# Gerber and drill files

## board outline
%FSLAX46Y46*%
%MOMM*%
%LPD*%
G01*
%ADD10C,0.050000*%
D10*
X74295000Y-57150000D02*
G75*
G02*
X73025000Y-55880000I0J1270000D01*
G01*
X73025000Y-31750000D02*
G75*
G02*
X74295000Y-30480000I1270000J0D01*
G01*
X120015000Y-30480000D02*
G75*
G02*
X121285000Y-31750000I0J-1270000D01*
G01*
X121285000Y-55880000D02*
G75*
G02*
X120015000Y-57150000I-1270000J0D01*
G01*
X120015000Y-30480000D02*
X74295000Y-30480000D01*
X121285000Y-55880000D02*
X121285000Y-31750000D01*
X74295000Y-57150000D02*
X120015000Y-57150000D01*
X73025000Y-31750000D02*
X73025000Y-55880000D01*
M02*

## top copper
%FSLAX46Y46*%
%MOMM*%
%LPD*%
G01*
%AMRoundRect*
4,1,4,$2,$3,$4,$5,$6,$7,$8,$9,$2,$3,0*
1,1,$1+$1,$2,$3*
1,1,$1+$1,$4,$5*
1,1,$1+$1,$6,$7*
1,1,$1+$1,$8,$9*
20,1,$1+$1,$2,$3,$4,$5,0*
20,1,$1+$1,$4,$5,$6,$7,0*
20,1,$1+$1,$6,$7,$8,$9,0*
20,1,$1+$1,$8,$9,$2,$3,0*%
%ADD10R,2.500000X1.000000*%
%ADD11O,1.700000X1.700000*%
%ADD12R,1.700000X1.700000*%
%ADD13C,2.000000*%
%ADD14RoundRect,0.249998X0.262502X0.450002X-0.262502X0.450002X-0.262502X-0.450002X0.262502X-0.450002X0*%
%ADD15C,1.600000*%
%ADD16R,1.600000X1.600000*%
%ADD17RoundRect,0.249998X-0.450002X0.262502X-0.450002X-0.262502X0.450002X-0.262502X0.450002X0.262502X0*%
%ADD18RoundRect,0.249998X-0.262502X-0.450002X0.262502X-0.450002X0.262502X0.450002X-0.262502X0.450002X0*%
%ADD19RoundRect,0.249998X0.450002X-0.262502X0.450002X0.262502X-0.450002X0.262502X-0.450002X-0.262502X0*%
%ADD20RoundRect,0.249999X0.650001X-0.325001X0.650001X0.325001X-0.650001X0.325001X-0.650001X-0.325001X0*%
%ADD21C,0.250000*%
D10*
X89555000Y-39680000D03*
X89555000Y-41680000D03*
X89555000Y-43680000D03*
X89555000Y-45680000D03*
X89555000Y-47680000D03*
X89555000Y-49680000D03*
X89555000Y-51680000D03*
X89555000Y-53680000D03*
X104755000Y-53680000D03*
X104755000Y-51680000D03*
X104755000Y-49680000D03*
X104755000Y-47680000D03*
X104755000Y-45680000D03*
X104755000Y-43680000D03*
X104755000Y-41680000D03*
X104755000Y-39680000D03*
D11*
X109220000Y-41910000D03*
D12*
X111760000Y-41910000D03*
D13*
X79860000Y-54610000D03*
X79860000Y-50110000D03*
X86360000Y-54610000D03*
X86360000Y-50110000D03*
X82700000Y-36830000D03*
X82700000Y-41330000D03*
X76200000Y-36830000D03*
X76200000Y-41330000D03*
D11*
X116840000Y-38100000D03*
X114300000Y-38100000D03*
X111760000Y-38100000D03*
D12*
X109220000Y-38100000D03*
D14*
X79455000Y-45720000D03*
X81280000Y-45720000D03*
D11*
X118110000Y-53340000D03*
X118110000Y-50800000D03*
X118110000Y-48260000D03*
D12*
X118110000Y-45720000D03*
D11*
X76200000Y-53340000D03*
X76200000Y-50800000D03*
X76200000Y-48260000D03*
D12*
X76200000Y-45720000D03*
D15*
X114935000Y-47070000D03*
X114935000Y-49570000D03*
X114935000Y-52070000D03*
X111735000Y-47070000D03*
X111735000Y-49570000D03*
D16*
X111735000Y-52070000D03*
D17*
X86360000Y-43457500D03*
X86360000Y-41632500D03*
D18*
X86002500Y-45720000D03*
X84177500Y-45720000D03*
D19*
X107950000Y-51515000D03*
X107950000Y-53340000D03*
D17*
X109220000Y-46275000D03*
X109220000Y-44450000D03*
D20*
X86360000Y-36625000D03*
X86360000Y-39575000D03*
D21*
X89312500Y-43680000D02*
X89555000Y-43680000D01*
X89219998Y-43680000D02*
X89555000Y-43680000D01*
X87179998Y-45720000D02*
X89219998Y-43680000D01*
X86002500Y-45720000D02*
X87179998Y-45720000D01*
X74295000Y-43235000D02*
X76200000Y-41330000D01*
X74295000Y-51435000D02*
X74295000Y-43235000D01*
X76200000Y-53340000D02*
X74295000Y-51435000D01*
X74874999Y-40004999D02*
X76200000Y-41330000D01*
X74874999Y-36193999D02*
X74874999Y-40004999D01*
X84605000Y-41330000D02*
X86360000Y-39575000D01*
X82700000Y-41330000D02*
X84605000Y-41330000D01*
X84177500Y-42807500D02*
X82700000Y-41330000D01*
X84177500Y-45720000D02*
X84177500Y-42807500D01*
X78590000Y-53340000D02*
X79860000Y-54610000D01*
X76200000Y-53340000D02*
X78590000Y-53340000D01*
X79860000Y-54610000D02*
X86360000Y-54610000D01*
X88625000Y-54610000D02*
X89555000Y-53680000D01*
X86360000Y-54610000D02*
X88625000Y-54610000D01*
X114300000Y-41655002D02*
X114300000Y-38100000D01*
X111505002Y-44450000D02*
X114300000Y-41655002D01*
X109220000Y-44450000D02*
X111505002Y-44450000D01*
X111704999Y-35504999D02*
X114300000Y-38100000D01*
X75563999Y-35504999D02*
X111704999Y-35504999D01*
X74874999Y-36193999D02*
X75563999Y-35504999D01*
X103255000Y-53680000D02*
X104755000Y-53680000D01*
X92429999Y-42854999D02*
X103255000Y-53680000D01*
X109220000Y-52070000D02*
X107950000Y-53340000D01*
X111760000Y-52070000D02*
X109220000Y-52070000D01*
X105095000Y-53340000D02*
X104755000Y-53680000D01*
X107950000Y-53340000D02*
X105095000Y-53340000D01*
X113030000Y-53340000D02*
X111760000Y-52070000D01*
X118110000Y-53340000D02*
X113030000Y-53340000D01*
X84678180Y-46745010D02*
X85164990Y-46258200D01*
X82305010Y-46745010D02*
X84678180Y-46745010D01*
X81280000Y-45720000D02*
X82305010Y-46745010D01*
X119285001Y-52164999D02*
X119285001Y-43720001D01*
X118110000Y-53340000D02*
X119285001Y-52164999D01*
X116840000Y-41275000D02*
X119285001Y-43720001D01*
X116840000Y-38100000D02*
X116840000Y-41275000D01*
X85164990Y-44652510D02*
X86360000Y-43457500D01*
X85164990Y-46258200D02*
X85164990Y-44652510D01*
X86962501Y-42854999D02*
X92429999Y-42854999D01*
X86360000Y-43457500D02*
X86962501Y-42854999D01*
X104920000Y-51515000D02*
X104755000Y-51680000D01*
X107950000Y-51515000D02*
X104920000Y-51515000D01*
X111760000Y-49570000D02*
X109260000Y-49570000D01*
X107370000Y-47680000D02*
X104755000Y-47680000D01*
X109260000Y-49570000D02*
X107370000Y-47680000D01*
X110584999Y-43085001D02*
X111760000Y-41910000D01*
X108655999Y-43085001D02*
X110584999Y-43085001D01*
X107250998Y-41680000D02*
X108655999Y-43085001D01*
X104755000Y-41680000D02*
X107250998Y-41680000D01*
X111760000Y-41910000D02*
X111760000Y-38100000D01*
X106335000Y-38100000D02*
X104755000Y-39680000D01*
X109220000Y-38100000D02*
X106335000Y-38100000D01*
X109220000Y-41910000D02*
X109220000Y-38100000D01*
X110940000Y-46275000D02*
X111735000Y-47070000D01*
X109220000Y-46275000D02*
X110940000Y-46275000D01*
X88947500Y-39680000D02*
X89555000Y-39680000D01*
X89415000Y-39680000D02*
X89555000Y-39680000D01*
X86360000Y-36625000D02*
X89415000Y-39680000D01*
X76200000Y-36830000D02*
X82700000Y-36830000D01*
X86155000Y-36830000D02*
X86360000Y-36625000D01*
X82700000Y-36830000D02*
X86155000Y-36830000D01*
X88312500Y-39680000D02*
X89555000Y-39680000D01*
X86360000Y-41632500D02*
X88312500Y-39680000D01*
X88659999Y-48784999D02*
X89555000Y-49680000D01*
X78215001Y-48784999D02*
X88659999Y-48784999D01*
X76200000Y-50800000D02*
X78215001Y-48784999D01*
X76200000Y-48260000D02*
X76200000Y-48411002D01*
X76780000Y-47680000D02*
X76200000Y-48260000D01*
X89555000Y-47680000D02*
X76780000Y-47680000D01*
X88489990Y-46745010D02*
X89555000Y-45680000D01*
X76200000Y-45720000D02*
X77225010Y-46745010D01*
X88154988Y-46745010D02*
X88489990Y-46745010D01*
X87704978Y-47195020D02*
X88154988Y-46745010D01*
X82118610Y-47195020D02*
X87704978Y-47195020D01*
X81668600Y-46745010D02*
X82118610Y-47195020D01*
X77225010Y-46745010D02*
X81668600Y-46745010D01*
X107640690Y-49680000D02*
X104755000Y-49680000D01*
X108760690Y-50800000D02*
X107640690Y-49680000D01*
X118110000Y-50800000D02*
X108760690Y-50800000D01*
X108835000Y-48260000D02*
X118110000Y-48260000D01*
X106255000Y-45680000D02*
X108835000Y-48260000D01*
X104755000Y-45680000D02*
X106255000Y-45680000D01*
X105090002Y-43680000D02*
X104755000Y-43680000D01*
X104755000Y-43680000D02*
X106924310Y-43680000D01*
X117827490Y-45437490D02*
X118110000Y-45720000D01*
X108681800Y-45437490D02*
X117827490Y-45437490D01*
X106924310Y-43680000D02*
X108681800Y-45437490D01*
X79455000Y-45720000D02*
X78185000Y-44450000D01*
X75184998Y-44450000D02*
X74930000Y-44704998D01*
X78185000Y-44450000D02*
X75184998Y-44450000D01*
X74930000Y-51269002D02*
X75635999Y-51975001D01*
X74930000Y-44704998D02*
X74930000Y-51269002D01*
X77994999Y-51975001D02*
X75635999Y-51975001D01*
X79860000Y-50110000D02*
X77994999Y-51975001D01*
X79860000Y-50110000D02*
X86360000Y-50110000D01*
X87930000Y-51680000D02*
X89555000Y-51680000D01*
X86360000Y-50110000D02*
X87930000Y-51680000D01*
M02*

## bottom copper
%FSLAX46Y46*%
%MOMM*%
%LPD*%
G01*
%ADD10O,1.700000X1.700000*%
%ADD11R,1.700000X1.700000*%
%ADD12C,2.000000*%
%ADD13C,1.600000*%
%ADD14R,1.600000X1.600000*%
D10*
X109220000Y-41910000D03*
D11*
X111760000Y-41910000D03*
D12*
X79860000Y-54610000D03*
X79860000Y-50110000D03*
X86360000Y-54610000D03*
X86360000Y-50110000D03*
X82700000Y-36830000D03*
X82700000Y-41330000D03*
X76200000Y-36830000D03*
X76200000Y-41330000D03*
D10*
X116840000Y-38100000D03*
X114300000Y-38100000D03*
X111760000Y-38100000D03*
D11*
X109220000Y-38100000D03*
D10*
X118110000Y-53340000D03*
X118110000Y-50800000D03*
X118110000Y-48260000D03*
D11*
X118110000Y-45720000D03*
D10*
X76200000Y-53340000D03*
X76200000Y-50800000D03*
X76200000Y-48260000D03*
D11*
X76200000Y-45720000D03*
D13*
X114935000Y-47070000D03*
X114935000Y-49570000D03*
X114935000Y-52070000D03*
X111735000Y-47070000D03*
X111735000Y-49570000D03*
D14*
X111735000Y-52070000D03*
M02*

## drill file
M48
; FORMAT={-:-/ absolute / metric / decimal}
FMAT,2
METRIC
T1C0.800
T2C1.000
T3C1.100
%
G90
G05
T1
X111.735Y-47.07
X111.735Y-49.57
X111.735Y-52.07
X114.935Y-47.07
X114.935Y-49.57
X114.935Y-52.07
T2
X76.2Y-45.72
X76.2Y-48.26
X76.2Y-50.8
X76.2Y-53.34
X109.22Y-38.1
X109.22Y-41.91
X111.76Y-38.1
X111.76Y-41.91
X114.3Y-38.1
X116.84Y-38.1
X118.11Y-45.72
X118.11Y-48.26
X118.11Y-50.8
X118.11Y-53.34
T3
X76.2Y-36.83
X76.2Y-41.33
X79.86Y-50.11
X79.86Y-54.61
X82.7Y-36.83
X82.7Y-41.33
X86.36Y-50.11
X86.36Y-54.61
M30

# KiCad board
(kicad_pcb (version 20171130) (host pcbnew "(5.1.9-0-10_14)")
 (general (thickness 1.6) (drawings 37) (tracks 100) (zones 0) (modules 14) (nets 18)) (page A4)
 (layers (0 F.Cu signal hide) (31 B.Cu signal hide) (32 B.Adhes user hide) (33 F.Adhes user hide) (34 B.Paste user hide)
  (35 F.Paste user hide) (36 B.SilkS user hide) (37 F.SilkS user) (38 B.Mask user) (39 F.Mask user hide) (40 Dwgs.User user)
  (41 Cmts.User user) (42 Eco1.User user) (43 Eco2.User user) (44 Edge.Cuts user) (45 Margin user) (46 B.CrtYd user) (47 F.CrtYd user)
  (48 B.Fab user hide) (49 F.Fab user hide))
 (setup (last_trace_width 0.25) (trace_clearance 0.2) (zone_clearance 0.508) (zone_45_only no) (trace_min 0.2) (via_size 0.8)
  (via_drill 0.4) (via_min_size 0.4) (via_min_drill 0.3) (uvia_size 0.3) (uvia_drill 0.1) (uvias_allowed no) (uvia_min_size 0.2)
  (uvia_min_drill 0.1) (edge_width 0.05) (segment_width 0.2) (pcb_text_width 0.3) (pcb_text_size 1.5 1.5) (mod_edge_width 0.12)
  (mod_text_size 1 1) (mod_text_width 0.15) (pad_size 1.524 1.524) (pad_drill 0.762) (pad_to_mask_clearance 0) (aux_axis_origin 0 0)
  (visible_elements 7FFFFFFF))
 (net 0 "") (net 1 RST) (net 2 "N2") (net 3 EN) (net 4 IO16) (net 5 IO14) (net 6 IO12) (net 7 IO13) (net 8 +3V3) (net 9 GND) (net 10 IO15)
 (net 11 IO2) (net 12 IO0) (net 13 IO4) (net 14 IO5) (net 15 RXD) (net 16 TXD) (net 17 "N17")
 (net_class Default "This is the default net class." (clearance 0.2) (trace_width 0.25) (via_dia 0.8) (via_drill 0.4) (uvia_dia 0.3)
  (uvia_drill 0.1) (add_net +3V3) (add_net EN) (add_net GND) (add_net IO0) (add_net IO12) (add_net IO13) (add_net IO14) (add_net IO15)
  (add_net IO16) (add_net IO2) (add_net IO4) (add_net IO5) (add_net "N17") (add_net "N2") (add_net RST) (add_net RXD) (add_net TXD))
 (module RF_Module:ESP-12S (layer F.Cu) (at 97.155 43.18)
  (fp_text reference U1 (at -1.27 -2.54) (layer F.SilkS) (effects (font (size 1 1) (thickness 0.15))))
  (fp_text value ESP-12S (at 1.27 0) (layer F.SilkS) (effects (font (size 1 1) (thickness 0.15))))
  (pad 1 smd rect (at -7.6 -3.5) (size 2.5 1) (layers F.Cu F.Paste F.Mask) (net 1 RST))
  (pad 2 smd rect (at -7.6 -1.5) (size 2.5 1) (layers F.Cu F.Paste F.Mask) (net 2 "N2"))
  (pad 3 smd rect (at -7.6 0.5) (size 2.5 1) (layers F.Cu F.Paste F.Mask) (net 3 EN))
  (pad 4 smd rect (at -7.6 2.5) (size 2.5 1) (layers F.Cu F.Paste F.Mask) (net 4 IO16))
  (pad 5 smd rect (at -7.6 4.5) (size 2.5 1) (layers F.Cu F.Paste F.Mask) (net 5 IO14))
  (pad 6 smd rect (at -7.6 6.5) (size 2.5 1) (layers F.Cu F.Paste F.Mask) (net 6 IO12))
  (pad 7 smd rect (at -7.6 8.5) (size 2.5 1) (layers F.Cu F.Paste F.Mask) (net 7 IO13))
  (pad 8 smd rect (at -7.6 10.5) (size 2.5 1) (layers F.Cu F.Paste F.Mask) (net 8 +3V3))
  (pad 9 smd rect (at 7.6 10.5) (size 2.5 1) (layers F.Cu F.Paste F.Mask) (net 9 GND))
  (pad 10 smd rect (at 7.6 8.5) (size 2.5 1) (layers F.Cu F.Paste F.Mask) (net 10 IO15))
  (pad 11 smd rect (at 7.6 6.5) (size 2.5 1) (layers F.Cu F.Paste F.Mask) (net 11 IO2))
  (pad 12 smd rect (at 7.6 4.5) (size 2.5 1) (layers F.Cu F.Paste F.Mask) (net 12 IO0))
  (pad 13 smd rect (at 7.6 2.5) (size 2.5 1) (layers F.Cu F.Paste F.Mask) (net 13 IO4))
  (pad 14 smd rect (at 7.6 0.5) (size 2.5 1) (layers F.Cu F.Paste F.Mask) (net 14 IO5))
  (pad 15 smd rect (at 7.6 -1.5) (size 2.5 1) (layers F.Cu F.Paste F.Mask) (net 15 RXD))
  (pad 16 smd rect (at 7.6 -3.5) (size 2.5 1) (layers F.Cu F.Paste F.Mask) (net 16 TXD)))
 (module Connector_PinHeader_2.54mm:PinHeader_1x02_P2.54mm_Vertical (layer B.Cu) (at 111.76 41.91 90)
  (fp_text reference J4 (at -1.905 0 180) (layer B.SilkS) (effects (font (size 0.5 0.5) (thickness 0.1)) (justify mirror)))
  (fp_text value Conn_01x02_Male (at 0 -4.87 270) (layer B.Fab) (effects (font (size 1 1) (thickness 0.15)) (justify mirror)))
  (pad 2 thru_hole oval (at 0 -2.54 90) (size 1.7 1.7) (drill 1) (layers *.Cu *.Mask) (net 16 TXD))
  (pad 1 thru_hole rect (at 0 0 90) (size 1.7 1.7) (drill 1) (layers *.Cu *.Mask) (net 15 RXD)))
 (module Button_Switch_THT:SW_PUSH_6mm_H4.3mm (layer F.Cu) (at 86.36 54.61 180)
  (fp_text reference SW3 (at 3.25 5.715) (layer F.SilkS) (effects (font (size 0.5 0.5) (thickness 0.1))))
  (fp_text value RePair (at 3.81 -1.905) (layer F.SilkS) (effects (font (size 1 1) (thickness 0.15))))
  (pad 1 thru_hole circle (at 6.5 0 270) (size 2 2) (drill 1.1) (layers *.Cu *.Mask) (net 8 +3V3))
  (pad 2 thru_hole circle (at 6.5 4.5 270) (size 2 2) (drill 1.1) (layers *.Cu *.Mask) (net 7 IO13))
  (pad 1 thru_hole circle (at 0 0 270) (size 2 2) (drill 1.1) (layers *.Cu *.Mask) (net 8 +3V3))
  (pad 2 thru_hole circle (at 0 4.5 270) (size 2 2) (drill 1.1) (layers *.Cu *.Mask) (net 7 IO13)))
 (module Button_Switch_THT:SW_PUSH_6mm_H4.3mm (layer F.Cu) (at 76.2 36.83)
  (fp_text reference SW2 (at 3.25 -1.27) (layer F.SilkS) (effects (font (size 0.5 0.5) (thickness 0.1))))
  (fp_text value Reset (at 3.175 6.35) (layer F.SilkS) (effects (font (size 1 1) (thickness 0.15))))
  (pad 1 thru_hole circle (at 6.5 0 90) (size 2 2) (drill 1.1) (layers *.Cu *.Mask) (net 1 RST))
  (pad 2 thru_hole circle (at 6.5 4.5 90) (size 2 2) (drill 1.1) (layers *.Cu *.Mask) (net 8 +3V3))
  (pad 1 thru_hole circle (at 0 0 90) (size 2 2) (drill 1.1) (layers *.Cu *.Mask) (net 1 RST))
  (pad 2 thru_hole circle (at 0 4.5 90) (size 2 2) (drill 1.1) (layers *.Cu *.Mask) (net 8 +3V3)))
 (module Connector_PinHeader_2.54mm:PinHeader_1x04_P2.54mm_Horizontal (layer F.Cu) (at 109.22 38.1 90)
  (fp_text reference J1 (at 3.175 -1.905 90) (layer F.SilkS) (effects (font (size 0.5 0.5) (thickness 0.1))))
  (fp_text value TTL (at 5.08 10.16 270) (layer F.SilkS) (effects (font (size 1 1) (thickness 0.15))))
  (pad 4 thru_hole oval (at 0 7.62 90) (size 1.7 1.7) (drill 1) (layers *.Cu *.Mask) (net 9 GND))
  (pad 3 thru_hole oval (at 0 5.08 90) (size 1.7 1.7) (drill 1) (layers *.Cu *.Mask) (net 8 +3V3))
  (pad 2 thru_hole oval (at 0 2.54 90) (size 1.7 1.7) (drill 1) (layers *.Cu *.Mask) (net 15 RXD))
  (pad 1 thru_hole rect (at 0 0 90) (size 1.7 1.7) (drill 1) (layers *.Cu *.Mask) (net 16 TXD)))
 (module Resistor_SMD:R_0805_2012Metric (layer F.Cu) (at 80.3675 45.72 180)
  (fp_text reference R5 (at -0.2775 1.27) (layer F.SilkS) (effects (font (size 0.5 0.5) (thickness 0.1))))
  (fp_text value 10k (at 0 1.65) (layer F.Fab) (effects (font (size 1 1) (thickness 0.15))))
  (pad 2 smd roundrect (at 0.9125 0 180) (size 1.025 1.4) (layers F.Cu F.Paste F.Mask) (roundrect_rratio 0.2439004878048781) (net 7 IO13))
  (pad 1 smd roundrect (at -0.9125 0 180) (size 1.025 1.4) (layers F.Cu F.Paste F.Mask) (roundrect_rratio 0.2439004878048781) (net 9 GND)))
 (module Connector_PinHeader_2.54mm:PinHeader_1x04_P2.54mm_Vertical (layer B.Cu) (at 118.11 45.72 180)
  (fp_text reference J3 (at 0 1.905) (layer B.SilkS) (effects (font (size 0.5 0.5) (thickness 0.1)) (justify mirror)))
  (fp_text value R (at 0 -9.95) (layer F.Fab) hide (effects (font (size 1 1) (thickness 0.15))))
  (pad 4 thru_hole oval (at 0 -7.62 180) (size 1.7 1.7) (drill 1) (layers *.Cu *.Mask) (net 9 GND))
  (pad 3 thru_hole oval (at 0 -5.08 180) (size 1.7 1.7) (drill 1) (layers *.Cu *.Mask) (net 11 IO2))
  (pad 2 thru_hole oval (at 0 -2.54 180) (size 1.7 1.7) (drill 1) (layers *.Cu *.Mask) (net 13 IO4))
  (pad 1 thru_hole rect (at 0 0 180) (size 1.7 1.7) (drill 1) (layers *.Cu *.Mask) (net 14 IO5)))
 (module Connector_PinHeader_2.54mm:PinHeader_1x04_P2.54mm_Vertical (layer B.Cu) (at 76.2 45.72 180)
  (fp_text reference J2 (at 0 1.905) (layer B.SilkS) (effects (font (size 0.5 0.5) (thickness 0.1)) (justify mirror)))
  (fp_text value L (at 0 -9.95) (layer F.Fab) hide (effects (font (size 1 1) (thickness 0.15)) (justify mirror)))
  (pad 4 thru_hole oval (at 0 -7.62 180) (size 1.7 1.7) (drill 1) (layers *.Cu *.Mask) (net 8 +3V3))
  (pad 3 thru_hole oval (at 0 -5.08 180) (size 1.7 1.7) (drill 1) (layers *.Cu *.Mask) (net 6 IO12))
  (pad 2 thru_hole oval (at 0 -2.54 180) (size 1.7 1.7) (drill 1) (layers *.Cu *.Mask) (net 5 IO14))
  (pad 1 thru_hole rect (at 0 0 180) (size 1.7 1.7) (drill 1) (layers *.Cu *.Mask) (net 4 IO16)))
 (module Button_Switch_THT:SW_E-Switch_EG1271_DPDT (layer F.Cu) (at 111.735 52.07 90)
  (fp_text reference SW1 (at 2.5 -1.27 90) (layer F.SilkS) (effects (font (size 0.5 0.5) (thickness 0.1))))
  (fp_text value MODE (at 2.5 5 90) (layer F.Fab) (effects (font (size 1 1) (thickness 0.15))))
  (pad 6 thru_hole circle (at 5 3.2 90) (size 1.6 1.6) (drill 0.8) (layers *.Cu *.Mask))
  (pad 5 thru_hole circle (at 2.5 3.2 90) (size 1.6 1.6) (drill 0.8) (layers *.Cu *.Mask))
  (pad 4 thru_hole circle (at 0 3.2 90) (size 1.6 1.6) (drill 0.8) (layers *.Cu *.Mask))
  (pad 3 thru_hole circle (at 5 0 90) (size 1.6 1.6) (drill 0.8) (layers *.Cu *.Mask) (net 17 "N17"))
  (pad 2 thru_hole circle (at 2.5 0 90) (size 1.6 1.6) (drill 0.8) (layers *.Cu *.Mask) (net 12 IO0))
  (pad 1 thru_hole rect (at 0 0 90) (size 1.6 1.6) (drill 0.8) (layers *.Cu *.Mask) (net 9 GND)))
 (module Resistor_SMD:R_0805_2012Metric (layer F.Cu) (at 86.36 42.545 270)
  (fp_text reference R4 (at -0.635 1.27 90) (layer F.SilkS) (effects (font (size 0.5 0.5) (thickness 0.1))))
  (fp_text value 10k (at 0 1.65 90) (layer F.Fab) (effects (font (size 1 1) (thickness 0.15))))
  (pad 2 smd roundrect (at 0.9125 0 270) (size 1.025 1.4) (layers F.Cu F.Paste F.Mask) (roundrect_rratio 0.2439004878048781) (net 9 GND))
  (pad 1 smd roundrect (at -0.9125 0 270) (size 1.025 1.4) (layers F.Cu F.Paste F.Mask) (roundrect_rratio 0.2439004878048781) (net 1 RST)))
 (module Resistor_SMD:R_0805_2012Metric (layer F.Cu) (at 85.09 45.72)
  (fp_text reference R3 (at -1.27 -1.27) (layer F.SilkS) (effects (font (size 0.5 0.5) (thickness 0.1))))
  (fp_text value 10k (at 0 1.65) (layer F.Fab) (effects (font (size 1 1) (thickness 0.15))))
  (pad 2 smd roundrect (at 0.9125 0) (size 1.025 1.4) (layers F.Cu F.Paste F.Mask) (roundrect_rratio 0.2439004878048781) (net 3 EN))
  (pad 1 smd roundrect (at -0.9125 0) (size 1.025 1.4) (layers F.Cu F.Paste F.Mask) (roundrect_rratio 0.2439004878048781) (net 8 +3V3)))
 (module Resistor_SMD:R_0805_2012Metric (layer F.Cu) (at 107.95 52.4275 90)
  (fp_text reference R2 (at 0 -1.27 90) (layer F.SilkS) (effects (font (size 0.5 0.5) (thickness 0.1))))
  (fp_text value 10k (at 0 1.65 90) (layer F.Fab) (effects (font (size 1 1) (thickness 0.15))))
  (pad 2 smd roundrect (at 0.9125 0 90) (size 1.025 1.4) (layers F.Cu F.Paste F.Mask) (roundrect_rratio 0.2439004878048781) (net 10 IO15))
  (pad 1 smd roundrect (at -0.9125 0 90) (size 1.025 1.4) (layers F.Cu F.Paste F.Mask) (roundrect_rratio 0.2439004878048781) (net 9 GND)))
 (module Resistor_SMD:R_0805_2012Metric (layer F.Cu) (at 109.22 45.3625 270)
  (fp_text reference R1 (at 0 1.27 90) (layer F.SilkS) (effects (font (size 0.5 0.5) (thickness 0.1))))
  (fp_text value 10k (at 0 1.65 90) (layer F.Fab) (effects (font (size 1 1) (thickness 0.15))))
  (pad 2 smd roundrect (at 0.9125 0 270) (size 1.025 1.4) (layers F.Cu F.Paste F.Mask) (roundrect_rratio 0.2439004878048781) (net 17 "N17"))
  (pad 1 smd roundrect (at -0.9125 0 270) (size 1.025 1.4) (layers F.Cu F.Paste F.Mask) (roundrect_rratio 0.2439004878048781) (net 8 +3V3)))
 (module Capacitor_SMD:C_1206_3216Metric (layer F.Cu) (at 86.36 38.1 90)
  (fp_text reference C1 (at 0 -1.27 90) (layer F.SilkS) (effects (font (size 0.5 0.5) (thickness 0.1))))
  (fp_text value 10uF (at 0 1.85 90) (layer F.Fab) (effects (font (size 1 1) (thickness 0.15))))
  (pad 2 smd roundrect (at 1.475 0 90) (size 1.15 1.8) (layers F.Cu F.Paste F.Mask) (roundrect_rratio 0.2173904347826087) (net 1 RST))
  (pad 1 smd roundrect (at -1.475 0 90) (size 1.15 1.8) (layers F.Cu F.Paste F.Mask) (roundrect_rratio 0.2173904347826087) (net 8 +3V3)))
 (gr_arc (start 74.295 55.88) (end 73.025 55.88) (angle -90) (layer Edge.Cuts) (width 0.05))
 (gr_arc (start 74.295 31.75) (end 74.295 30.48) (angle -90) (layer Edge.Cuts) (width 0.05))
 (gr_arc (start 120.015 31.75) (end 121.285 31.75) (angle -90) (layer Edge.Cuts) (width 0.05))
 (gr_arc (start 120.015 55.88) (end 120.015 57.15) (angle -90) (layer Edge.Cuts) (width 0.05))
 (gr_line (start 120.015 30.48) (end 74.295 30.48) (layer Edge.Cuts) (width 0.05))
 (gr_line (start 121.285 55.88) (end 121.285 31.75) (layer Edge.Cuts) (width 0.05))
 (gr_line (start 74.295 57.15) (end 120.015 57.15) (layer Edge.Cuts) (width 0.05))
 (gr_line (start 73.025 31.75) (end 73.025 55.88) (layer Edge.Cuts) (width 0.05))
 (segment (start 89.3125 43.68) (end 89.555 43.68) (width 0.25) (layer F.Cu) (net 3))
 (segment (start 89.219998 43.68) (end 89.555 43.68) (width 0.25) (layer F.Cu) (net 3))
 (segment (start 87.179998 45.72) (end 89.219998 43.68) (width 0.25) (layer F.Cu) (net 3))
 (segment (start 86.0025 45.72) (end 87.179998 45.72) (width 0.25) (layer F.Cu) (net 3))
 (segment (start 74.295 43.235) (end 76.2 41.33) (width 0.25) (layer F.Cu) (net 8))
 (segment (start 74.295 51.435) (end 74.295 43.235) (width 0.25) (layer F.Cu) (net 8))
 (segment (start 76.2 53.34) (end 74.295 51.435) (width 0.25) (layer F.Cu) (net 8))
 (segment (start 74.874999 40.004999) (end 76.2 41.33) (width 0.25) (layer F.Cu) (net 8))
 (segment (start 74.874999 36.193999) (end 74.874999 40.004999) (width 0.25) (layer F.Cu) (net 8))
 (segment (start 84.605 41.33) (end 86.36 39.575) (width 0.25) (layer F.Cu) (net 8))
 (segment (start 82.7 41.33) (end 84.605 41.33) (width 0.25) (layer F.Cu) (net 8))
 (segment (start 84.1775 42.8075) (end 82.7 41.33) (width 0.25) (layer F.Cu) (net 8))
 (segment (start 84.1775 45.72) (end 84.1775 42.8075) (width 0.25) (layer F.Cu) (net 8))
 (segment (start 78.59 53.34) (end 79.86 54.61) (width 0.25) (layer F.Cu) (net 8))
 (segment (start 76.2 53.34) (end 78.59 53.34) (width 0.25) (layer F.Cu) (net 8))
 (segment (start 79.86 54.61) (end 86.36 54.61) (width 0.25) (layer F.Cu) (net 8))
 (segment (start 88.625 54.61) (end 89.555 53.68) (width 0.25) (layer F.Cu) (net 8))
 (segment (start 86.36 54.61) (end 88.625 54.61) (width 0.25) (layer F.Cu) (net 8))
 (segment (start 114.3 41.655002) (end 114.3 38.1) (width 0.25) (layer F.Cu) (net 8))
 (segment (start 111.505002 44.45) (end 114.3 41.655002) (width 0.25) (layer F.Cu) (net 8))
 (segment (start 109.22 44.45) (end 111.505002 44.45) (width 0.25) (layer F.Cu) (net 8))
 (segment (start 111.704999 35.504999) (end 114.3 38.1) (width 0.25) (layer F.Cu) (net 8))
 (segment (start 75.563999 35.504999) (end 111.704999 35.504999) (width 0.25) (layer F.Cu) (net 8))
 (segment (start 74.874999 36.193999) (end 75.563999 35.504999) (width 0.25) (layer F.Cu) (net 8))
 (segment (start 103.255 53.68) (end 104.755 53.68) (width 0.25) (layer F.Cu) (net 9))
 (segment (start 92.429999 42.854999) (end 103.255 53.68) (width 0.25) (layer F.Cu) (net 9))
 (segment (start 109.22 52.07) (end 107.95 53.34) (width 0.25) (layer F.Cu) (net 9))
 (segment (start 111.76 52.07) (end 109.22 52.07) (width 0.25) (layer F.Cu) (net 9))
 (segment (start 105.095 53.34) (end 104.755 53.68) (width 0.25) (layer F.Cu) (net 9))
 (segment (start 107.95 53.34) (end 105.095 53.34) (width 0.25) (layer F.Cu) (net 9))
 (segment (start 113.03 53.34) (end 111.76 52.07) (width 0.25) (layer F.Cu) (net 9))
 (segment (start 118.11 53.34) (end 113.03 53.34) (width 0.25) (layer F.Cu) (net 9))
 (segment (start 84.67818 46.74501) (end 85.16499 46.2582) (width 0.25) (layer F.Cu) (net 9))
 (segment (start 82.30501 46.74501) (end 84.67818 46.74501) (width 0.25) (layer F.Cu) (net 9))
 (segment (start 81.28 45.72) (end 82.30501 46.74501) (width 0.25) (layer F.Cu) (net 9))
 (segment (start 119.285001 52.164999) (end 119.285001 43.720001) (width 0.25) (layer F.Cu) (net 9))
 (segment (start 118.11 53.34) (end 119.285001 52.164999) (width 0.25) (layer F.Cu) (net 9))
 (segment (start 116.84 41.275) (end 119.285001 43.720001) (width 0.25) (layer F.Cu) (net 9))
 (segment (start 116.84 38.1) (end 116.84 41.275) (width 0.25) (layer F.Cu) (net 9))
 (segment (start 85.16499 44.65251) (end 86.36 43.4575) (width 0.25) (layer F.Cu) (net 9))
 (segment (start 85.16499 46.2582) (end 85.16499 44.65251) (width 0.25) (layer F.Cu) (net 9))
 (segment (start 86.962501 42.854999) (end 92.429999 42.854999) (width 0.25) (layer F.Cu) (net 9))
 (segment (start 86.36 43.4575) (end 86.962501 42.854999) (width 0.25) (layer F.Cu) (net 9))
 (segment (start 104.92 51.515) (end 104.755 51.68) (width 0.25) (layer F.Cu) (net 10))
 (segment (start 107.95 51.515) (end 104.92 51.515) (width 0.25) (layer F.Cu) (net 10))
 (segment (start 111.76 49.57) (end 109.26 49.57) (width 0.25) (layer F.Cu) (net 12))
 (segment (start 107.37 47.68) (end 104.755 47.68) (width 0.25) (layer F.Cu) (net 12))
 (segment (start 109.26 49.57) (end 107.37 47.68) (width 0.25) (layer F.Cu) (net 12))
 (segment (start 110.584999 43.085001) (end 111.76 41.91) (width 0.25) (layer F.Cu) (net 15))
 (segment (start 108.655999 43.085001) (end 110.584999 43.085001) (width 0.25) (layer F.Cu) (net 15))
 (segment (start 107.250998 41.68) (end 108.655999 43.085001) (width 0.25) (layer F.Cu) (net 15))
 (segment (start 104.755 41.68) (end 107.250998 41.68) (width 0.25) (layer F.Cu) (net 15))
 (segment (start 111.76 41.91) (end 111.76 38.1) (width 0.25) (layer F.Cu) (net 15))
 (segment (start 106.335 38.1) (end 104.755 39.68) (width 0.25) (layer F.Cu) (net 16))
 (segment (start 109.22 38.1) (end 106.335 38.1) (width 0.25) (layer F.Cu) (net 16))
 (segment (start 109.22 41.91) (end 109.22 38.1) (width 0.25) (layer F.Cu) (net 16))
 (segment (start 110.94 46.275) (end 111.735 47.07) (width 0.25) (layer F.Cu) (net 17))
 (segment (start 109.22 46.275) (end 110.94 46.275) (width 0.25) (layer F.Cu) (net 17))
 (segment (start 88.9475 39.68) (end 89.555 39.68) (width 0.25) (layer F.Cu) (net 1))
 (segment (start 89.415 39.68) (end 89.555 39.68) (width 0.25) (layer F.Cu) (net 1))
 (segment (start 86.36 36.625) (end 89.415 39.68) (width 0.25) (layer F.Cu) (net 1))
 (segment (start 76.2 36.83) (end 82.7 36.83) (width 0.25) (layer F.Cu) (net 1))
 (segment (start 86.155 36.83) (end 86.36 36.625) (width 0.25) (layer F.Cu) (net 1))
 (segment (start 82.7 36.83) (end 86.155 36.83) (width 0.25) (layer F.Cu) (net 1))
 (segment (start 88.3125 39.68) (end 89.555 39.68) (width 0.25) (layer F.Cu) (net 1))
 (segment (start 86.36 41.6325) (end 88.3125 39.68) (width 0.25) (layer F.Cu) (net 1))
 (segment (start 88.659999 48.784999) (end 89.555 49.68) (width 0.25) (layer F.Cu) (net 6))
 (segment (start 78.215001 48.784999) (end 88.659999 48.784999) (width 0.25) (layer F.Cu) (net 6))
 (segment (start 76.2 50.8) (end 78.215001 48.784999) (width 0.25) (layer F.Cu) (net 6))
 (segment (start 76.2 48.26) (end 76.2 48.411002) (width 0.25) (layer F.Cu) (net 5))
 (segment (start 76.78 47.68) (end 76.2 48.26) (width 0.25) (layer F.Cu) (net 5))
 (segment (start 89.555 47.68) (end 76.78 47.68) (width 0.25) (layer F.Cu) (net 5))
 (segment (start 88.48999 46.74501) (end 89.555 45.68) (width 0.25) (layer F.Cu) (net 4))
 (segment (start 76.2 45.72) (end 77.22501 46.74501) (width 0.25) (layer F.Cu) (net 4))
 (segment (start 88.154988 46.74501) (end 88.48999 46.74501) (width 0.25) (layer F.Cu) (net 4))
 (segment (start 87.704978 47.19502) (end 88.154988 46.74501) (width 0.25) (layer F.Cu) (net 4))
 (segment (start 82.11861 47.19502) (end 87.704978 47.19502) (width 0.25) (layer F.Cu) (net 4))
 (segment (start 81.6686 46.74501) (end 82.11861 47.19502) (width 0.25) (layer F.Cu) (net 4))
 (segment (start 77.22501 46.74501) (end 81.6686 46.74501) (width 0.25) (layer F.Cu) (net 4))
 (segment (start 107.64069 49.68) (end 104.755 49.68) (width 0.25) (layer F.Cu) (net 11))
 (segment (start 108.76069 50.8) (end 107.64069 49.68) (width 0.25) (layer F.Cu) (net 11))
 (segment (start 118.11 50.8) (end 108.76069 50.8) (width 0.25) (layer F.Cu) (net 11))
 (segment (start 108.835 48.26) (end 118.11 48.26) (width 0.25) (layer F.Cu) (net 13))
 (segment (start 106.255 45.68) (end 108.835 48.26) (width 0.25) (layer F.Cu) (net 13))
 (segment (start 104.755 45.68) (end 106.255 45.68) (width 0.25) (layer F.Cu) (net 13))
 (segment (start 105.090002 43.68) (end 104.755 43.68) (width 0.25) (layer F.Cu) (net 14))
 (segment (start 104.755 43.68) (end 106.92431 43.68) (width 0.25) (layer F.Cu) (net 14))
 (segment (start 117.82749 45.43749) (end 118.11 45.72) (width 0.25) (layer F.Cu) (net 14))
 (segment (start 108.6818 45.43749) (end 117.82749 45.43749) (width 0.25) (layer F.Cu) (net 14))
 (segment (start 106.92431 43.68) (end 108.6818 45.43749) (width 0.25) (layer F.Cu) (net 14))
 (segment (start 79.455 45.72) (end 78.185 44.45) (width 0.25) (layer F.Cu) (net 7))
 (segment (start 75.184998 44.45) (end 74.93 44.704998) (width 0.25) (layer F.Cu) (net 7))
 (segment (start 78.185 44.45) (end 75.184998 44.45) (width 0.25) (layer F.Cu) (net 7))
 (segment (start 74.93 51.269002) (end 75.635999 51.975001) (width 0.25) (layer F.Cu) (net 7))
 (segment (start 74.93 44.704998) (end 74.93 51.269002) (width 0.25) (layer F.Cu) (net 7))
 (segment (start 77.994999 51.975001) (end 75.635999 51.975001) (width 0.25) (layer F.Cu) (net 7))
 (segment (start 79.86 50.11) (end 77.994999 51.975001) (width 0.25) (layer F.Cu) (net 7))
 (segment (start 79.86 50.11) (end 86.36 50.11) (width 0.25) (layer F.Cu) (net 7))
 (segment (start 87.93 51.68) (end 89.555 51.68) (width 0.25) (layer F.Cu) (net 7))
 (segment (start 86.36 50.11) (end 87.93 51.68) (width 0.25) (layer F.Cu) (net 7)))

